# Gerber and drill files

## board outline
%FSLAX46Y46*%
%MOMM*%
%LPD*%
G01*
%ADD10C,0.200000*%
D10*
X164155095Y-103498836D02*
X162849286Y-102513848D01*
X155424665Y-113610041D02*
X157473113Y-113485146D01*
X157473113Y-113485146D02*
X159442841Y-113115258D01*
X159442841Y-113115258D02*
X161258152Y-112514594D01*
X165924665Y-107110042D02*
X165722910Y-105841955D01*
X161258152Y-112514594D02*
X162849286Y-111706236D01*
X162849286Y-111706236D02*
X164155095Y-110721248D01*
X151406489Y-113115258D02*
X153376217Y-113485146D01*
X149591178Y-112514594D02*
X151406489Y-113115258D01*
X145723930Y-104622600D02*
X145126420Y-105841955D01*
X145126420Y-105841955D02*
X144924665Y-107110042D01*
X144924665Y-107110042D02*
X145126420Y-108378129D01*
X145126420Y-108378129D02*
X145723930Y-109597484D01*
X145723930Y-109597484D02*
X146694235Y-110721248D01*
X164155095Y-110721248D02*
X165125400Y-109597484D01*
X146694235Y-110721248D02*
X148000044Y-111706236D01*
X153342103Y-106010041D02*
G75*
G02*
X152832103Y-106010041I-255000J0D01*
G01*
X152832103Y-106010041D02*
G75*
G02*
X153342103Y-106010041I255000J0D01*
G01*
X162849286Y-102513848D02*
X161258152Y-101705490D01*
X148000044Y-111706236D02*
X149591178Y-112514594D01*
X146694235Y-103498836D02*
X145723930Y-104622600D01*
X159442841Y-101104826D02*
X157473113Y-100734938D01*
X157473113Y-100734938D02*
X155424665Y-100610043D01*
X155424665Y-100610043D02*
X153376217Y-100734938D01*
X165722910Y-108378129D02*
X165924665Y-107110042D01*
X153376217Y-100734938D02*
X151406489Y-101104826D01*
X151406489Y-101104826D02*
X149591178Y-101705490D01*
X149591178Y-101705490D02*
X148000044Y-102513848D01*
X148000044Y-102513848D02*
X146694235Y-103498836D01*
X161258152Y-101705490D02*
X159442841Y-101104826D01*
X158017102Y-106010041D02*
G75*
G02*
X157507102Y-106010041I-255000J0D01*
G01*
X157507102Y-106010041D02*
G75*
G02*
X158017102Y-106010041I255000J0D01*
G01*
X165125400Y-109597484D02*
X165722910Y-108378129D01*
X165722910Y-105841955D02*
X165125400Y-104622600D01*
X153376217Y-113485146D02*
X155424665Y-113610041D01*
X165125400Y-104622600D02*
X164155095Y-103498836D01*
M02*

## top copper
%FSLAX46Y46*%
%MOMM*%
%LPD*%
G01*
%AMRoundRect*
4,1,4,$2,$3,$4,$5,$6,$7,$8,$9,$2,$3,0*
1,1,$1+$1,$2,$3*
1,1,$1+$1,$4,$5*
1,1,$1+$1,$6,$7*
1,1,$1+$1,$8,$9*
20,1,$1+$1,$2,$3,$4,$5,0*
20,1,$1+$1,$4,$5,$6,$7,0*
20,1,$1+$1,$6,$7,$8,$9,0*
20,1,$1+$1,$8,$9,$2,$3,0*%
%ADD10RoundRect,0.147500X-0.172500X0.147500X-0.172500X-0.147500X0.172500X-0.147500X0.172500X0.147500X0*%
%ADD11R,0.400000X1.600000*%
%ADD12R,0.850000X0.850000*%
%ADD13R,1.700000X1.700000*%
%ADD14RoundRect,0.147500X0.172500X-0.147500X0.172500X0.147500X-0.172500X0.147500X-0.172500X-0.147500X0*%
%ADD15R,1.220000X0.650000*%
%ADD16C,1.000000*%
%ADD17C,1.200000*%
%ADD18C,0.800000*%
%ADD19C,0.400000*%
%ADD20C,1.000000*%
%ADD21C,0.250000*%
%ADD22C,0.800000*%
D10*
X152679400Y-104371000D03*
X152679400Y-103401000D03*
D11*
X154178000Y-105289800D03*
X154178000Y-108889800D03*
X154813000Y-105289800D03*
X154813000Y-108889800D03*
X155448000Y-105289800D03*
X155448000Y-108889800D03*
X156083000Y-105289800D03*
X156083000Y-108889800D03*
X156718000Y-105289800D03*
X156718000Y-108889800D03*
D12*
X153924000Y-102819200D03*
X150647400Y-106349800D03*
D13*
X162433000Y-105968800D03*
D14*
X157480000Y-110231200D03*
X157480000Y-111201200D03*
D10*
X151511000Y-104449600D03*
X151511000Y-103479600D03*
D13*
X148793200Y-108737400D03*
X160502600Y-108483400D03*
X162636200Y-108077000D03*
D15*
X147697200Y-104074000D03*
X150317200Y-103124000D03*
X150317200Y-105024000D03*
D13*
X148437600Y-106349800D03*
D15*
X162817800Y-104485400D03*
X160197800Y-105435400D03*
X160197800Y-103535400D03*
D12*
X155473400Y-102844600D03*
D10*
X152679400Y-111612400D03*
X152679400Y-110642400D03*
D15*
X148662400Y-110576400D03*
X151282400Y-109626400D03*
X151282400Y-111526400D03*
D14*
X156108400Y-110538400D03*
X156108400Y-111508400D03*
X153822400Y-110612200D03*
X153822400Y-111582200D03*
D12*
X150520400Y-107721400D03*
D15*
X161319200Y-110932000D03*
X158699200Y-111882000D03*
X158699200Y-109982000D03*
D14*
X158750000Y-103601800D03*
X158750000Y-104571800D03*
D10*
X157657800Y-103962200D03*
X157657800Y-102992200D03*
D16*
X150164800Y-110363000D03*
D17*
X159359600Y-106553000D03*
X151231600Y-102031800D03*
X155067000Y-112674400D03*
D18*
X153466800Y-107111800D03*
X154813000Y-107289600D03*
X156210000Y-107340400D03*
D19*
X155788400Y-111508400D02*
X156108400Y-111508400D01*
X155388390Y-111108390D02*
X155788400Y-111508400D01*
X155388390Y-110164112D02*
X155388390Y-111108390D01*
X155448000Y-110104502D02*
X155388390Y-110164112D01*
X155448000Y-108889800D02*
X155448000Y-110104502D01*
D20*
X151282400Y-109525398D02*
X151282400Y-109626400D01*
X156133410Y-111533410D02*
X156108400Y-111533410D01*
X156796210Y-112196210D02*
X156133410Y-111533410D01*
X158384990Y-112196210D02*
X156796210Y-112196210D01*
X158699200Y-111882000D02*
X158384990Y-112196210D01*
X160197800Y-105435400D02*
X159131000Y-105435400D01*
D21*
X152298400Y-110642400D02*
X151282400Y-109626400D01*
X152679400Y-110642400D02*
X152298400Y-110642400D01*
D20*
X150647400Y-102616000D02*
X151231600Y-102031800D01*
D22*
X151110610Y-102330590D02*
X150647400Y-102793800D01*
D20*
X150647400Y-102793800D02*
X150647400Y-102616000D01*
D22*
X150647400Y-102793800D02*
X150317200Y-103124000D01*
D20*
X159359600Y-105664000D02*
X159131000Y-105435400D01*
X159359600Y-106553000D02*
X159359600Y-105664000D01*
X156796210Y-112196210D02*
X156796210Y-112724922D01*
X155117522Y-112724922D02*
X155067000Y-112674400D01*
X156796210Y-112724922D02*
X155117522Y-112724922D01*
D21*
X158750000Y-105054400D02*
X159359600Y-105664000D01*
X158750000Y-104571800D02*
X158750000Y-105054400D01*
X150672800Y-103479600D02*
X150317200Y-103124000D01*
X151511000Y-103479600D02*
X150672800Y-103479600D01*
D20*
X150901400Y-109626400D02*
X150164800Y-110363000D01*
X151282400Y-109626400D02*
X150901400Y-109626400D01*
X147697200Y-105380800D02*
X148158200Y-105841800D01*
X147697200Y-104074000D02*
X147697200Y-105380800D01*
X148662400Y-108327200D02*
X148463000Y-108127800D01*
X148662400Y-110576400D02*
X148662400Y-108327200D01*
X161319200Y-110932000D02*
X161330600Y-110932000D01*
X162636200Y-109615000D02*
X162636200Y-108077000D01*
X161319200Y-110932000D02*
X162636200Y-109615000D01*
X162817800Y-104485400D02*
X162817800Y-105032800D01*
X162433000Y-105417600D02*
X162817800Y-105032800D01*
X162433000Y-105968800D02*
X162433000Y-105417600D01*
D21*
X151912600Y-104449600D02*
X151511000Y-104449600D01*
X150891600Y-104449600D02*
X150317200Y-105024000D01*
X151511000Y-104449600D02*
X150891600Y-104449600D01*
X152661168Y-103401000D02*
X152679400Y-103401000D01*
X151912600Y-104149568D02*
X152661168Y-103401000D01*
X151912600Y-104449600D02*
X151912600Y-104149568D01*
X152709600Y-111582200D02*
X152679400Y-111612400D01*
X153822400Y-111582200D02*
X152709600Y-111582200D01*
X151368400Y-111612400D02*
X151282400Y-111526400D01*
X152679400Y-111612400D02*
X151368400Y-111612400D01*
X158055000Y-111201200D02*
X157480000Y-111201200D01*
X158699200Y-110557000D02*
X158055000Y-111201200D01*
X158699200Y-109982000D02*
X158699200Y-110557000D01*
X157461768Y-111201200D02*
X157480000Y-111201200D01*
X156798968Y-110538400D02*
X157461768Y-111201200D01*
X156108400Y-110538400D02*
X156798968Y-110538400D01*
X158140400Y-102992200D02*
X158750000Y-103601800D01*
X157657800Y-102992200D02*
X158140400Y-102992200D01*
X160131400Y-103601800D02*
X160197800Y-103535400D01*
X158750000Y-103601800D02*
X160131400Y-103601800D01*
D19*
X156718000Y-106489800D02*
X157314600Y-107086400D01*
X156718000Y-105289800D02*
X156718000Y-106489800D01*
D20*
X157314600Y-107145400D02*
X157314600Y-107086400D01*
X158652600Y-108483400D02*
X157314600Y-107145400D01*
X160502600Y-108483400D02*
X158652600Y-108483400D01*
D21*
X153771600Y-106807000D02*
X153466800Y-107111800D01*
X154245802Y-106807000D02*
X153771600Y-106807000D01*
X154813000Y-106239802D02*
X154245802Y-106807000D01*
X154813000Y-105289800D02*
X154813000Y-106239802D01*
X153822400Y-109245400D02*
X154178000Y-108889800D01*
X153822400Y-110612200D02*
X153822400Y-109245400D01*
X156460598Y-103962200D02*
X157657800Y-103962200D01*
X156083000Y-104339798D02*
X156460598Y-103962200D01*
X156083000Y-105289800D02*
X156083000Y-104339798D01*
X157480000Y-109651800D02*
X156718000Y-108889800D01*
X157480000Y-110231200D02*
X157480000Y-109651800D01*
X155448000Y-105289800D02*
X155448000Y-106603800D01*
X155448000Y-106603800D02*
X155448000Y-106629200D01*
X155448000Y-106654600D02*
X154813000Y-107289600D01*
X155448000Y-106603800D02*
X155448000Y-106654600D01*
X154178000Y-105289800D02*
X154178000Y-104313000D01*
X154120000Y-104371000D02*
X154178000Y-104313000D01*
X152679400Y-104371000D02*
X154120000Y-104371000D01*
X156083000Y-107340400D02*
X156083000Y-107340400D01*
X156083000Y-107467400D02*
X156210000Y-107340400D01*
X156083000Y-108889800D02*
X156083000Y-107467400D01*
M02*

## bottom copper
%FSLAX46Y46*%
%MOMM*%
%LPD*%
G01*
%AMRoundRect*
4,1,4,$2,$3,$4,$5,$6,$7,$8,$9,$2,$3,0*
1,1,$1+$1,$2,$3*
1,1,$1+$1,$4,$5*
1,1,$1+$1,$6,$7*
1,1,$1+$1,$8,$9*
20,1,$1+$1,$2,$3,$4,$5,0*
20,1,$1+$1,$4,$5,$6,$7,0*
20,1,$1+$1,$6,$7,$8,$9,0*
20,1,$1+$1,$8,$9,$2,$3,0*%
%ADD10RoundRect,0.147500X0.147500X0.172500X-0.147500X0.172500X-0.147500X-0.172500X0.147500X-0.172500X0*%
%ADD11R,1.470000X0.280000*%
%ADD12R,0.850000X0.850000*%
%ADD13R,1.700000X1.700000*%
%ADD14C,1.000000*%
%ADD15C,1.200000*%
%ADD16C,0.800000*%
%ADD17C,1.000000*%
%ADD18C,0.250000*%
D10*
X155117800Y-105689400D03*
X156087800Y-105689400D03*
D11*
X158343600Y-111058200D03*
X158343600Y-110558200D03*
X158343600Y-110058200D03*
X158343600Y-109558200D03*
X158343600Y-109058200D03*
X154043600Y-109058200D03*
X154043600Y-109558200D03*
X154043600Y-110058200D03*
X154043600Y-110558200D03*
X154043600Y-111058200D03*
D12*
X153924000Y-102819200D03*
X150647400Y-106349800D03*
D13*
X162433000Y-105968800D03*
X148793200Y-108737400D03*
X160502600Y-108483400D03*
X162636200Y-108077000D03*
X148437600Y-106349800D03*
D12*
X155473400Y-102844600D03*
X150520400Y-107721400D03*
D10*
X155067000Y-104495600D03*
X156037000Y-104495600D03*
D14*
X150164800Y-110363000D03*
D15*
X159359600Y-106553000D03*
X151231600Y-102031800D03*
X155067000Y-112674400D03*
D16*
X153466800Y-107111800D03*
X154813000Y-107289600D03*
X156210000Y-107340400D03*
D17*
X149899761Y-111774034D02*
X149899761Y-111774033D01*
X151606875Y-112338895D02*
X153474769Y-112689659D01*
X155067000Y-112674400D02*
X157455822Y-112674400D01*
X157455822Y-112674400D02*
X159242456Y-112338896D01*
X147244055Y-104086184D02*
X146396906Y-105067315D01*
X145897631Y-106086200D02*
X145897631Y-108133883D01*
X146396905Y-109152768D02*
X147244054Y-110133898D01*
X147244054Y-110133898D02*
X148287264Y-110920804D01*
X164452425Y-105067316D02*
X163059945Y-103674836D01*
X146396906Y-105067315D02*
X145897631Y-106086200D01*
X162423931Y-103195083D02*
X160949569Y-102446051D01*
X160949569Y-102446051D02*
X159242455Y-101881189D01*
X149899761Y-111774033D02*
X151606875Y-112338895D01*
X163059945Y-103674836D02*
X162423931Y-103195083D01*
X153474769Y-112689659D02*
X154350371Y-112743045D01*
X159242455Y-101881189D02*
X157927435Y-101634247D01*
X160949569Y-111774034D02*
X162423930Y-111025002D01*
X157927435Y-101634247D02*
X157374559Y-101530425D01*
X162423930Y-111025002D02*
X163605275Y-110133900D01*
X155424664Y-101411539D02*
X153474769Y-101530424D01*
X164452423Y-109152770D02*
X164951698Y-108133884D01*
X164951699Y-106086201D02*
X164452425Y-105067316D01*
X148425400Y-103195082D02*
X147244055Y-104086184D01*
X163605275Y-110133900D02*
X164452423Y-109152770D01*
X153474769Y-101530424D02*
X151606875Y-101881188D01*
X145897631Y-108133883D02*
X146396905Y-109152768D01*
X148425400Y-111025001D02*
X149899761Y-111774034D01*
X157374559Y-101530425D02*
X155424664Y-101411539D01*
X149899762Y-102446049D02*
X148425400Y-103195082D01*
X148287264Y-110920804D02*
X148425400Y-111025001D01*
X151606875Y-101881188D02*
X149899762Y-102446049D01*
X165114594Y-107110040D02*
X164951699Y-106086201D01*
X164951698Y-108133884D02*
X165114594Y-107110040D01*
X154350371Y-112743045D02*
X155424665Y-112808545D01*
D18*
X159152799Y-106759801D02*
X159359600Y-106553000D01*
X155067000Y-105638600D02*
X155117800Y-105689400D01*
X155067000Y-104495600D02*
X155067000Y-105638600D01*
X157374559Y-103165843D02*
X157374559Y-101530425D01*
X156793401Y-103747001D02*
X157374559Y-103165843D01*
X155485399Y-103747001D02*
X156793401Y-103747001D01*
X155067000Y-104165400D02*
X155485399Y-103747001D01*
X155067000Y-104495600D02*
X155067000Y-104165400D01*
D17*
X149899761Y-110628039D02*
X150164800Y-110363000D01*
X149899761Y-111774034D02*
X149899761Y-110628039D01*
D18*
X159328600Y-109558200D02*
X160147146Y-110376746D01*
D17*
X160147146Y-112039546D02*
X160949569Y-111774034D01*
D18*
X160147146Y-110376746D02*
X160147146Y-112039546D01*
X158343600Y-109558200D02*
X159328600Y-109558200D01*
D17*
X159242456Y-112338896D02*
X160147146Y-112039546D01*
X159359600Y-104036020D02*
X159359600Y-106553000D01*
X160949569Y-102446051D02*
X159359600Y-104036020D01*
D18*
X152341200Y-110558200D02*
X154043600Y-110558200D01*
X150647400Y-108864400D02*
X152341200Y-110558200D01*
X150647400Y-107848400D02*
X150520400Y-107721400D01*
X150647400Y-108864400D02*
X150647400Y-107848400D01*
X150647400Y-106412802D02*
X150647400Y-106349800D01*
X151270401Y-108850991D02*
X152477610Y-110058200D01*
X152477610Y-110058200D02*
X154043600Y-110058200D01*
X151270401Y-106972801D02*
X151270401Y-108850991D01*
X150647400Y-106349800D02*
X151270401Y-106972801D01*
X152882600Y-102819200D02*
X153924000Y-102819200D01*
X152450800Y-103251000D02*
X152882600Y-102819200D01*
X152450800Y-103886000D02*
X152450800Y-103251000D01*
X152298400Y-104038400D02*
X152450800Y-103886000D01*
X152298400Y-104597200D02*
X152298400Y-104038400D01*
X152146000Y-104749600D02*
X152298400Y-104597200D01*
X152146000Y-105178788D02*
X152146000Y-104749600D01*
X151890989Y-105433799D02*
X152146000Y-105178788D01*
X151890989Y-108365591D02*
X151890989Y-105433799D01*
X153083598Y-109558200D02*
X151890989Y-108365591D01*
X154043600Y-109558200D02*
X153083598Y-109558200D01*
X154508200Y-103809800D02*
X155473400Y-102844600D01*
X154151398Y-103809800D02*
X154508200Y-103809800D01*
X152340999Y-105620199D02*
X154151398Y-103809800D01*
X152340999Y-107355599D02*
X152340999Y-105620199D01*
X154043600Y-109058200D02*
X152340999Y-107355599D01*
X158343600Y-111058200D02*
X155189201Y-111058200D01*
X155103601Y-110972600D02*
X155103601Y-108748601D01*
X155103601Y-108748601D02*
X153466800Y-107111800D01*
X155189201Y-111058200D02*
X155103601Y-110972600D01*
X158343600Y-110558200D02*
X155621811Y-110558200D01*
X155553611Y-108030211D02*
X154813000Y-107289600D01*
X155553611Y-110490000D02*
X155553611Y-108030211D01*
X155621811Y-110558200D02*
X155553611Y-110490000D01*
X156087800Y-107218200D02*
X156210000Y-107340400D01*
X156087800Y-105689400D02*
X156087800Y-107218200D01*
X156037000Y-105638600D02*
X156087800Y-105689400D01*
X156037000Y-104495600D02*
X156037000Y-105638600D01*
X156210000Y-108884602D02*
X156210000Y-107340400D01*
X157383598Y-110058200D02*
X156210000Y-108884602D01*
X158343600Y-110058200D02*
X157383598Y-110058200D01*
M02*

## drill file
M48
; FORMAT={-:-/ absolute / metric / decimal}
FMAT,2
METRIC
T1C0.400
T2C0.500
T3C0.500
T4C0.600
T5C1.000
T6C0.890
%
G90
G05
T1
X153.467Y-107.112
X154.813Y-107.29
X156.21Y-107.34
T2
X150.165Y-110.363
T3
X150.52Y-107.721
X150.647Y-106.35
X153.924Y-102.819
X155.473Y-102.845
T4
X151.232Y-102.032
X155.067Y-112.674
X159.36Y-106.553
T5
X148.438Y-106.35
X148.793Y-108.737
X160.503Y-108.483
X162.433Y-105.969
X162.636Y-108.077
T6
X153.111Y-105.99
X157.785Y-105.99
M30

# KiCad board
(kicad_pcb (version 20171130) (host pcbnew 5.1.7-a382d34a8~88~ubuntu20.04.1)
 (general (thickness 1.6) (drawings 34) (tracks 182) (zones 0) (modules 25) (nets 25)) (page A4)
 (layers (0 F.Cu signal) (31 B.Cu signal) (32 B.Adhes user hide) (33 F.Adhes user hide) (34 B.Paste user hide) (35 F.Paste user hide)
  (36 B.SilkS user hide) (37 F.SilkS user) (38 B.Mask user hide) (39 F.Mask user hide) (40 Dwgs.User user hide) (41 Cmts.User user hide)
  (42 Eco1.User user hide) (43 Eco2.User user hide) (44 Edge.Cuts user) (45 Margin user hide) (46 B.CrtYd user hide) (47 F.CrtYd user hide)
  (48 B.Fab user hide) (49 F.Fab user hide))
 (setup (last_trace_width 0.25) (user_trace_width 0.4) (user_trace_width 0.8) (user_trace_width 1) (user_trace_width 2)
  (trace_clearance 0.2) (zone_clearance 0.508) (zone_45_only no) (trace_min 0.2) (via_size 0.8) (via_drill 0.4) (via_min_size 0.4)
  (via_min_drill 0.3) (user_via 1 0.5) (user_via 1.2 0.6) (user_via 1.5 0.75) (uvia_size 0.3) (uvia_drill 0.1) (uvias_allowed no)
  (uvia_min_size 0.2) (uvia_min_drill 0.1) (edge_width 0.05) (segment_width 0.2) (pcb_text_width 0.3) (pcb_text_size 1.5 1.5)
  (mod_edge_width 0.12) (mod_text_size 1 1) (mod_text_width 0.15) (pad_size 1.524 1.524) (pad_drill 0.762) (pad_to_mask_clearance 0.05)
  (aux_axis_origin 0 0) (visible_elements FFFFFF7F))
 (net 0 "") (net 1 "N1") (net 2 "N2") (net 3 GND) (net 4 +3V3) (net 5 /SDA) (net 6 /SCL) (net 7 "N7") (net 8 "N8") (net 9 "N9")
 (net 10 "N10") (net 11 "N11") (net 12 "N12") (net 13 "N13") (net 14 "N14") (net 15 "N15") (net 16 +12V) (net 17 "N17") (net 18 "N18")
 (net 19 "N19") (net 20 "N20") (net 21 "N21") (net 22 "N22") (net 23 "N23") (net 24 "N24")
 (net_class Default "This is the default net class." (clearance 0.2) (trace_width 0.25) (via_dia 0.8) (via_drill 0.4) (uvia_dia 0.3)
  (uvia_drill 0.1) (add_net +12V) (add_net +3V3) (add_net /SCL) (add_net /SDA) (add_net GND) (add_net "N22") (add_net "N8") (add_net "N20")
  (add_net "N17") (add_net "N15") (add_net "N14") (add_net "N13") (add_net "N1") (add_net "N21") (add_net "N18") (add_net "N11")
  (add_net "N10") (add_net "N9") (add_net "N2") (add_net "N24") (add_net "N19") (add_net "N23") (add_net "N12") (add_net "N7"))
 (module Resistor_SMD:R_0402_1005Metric (layer F.Cu) (at 152.6794 103.886 270)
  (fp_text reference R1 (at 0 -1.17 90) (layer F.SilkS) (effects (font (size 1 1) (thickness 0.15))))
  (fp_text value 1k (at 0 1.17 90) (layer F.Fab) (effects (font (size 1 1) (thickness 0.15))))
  (pad 2 smd roundrect (at 0.485 0 270) (size 0.59 0.64) (layers F.Cu F.Paste F.Mask) (roundrect_rratio 0.25) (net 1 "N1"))
  (pad 1 smd roundrect (at -0.485 0 270) (size 0.59 0.64) (layers F.Cu F.Paste F.Mask) (roundrect_rratio 0.25) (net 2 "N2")))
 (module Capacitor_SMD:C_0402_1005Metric (layer B.Cu) (at 155.6028 105.6894 180)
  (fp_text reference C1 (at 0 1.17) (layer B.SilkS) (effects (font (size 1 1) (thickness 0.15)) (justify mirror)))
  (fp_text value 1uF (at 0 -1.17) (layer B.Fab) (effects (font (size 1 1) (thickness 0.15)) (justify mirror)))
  (pad 2 smd roundrect (at 0.485 0 180) (size 0.59 0.64) (layers B.Cu B.Paste B.Mask) (roundrect_rratio 0.25) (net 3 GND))
  (pad 1 smd roundrect (at -0.485 0 180) (size 0.59 0.64) (layers B.Cu B.Paste B.Mask) (roundrect_rratio 0.25) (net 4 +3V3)))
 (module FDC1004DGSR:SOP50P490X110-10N (layer B.Cu) (at 156.1936 110.0582)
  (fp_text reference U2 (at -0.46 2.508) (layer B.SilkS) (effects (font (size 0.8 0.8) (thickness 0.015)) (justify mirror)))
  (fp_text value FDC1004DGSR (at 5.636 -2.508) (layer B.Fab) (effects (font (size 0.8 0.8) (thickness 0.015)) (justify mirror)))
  (pad 10 smd rect (at 2.15 1) (size 1.47 0.28) (layers B.Cu B.Paste B.Mask) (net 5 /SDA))
  (pad 9 smd rect (at 2.15 0.5) (size 1.47 0.28) (layers B.Cu B.Paste B.Mask) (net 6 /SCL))
  (pad 8 smd rect (at 2.15 0) (size 1.47 0.28) (layers B.Cu B.Paste B.Mask) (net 4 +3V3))
  (pad 7 smd rect (at 2.15 -0.5) (size 1.47 0.28) (layers B.Cu B.Paste B.Mask) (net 3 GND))
  (pad 6 smd rect (at 2.15 -1) (size 1.47 0.28) (layers B.Cu B.Paste B.Mask) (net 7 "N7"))
  (pad 5 smd rect (at -2.15 -1) (size 1.47 0.28) (layers B.Cu B.Paste B.Mask) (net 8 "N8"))
  (pad 4 smd rect (at -2.15 -0.5) (size 1.47 0.28) (layers B.Cu B.Paste B.Mask) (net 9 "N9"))
  (pad 3 smd rect (at -2.15 0) (size 1.47 0.28) (layers B.Cu B.Paste B.Mask) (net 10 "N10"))
  (pad 2 smd rect (at -2.15 0.5) (size 1.47 0.28) (layers B.Cu B.Paste B.Mask) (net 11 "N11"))
  (pad 1 smd rect (at -2.15 1) (size 1.47 0.28) (layers B.Cu B.Paste B.Mask) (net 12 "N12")))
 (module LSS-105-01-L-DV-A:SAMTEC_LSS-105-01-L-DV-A (layer F.Cu) (at 156.718 108.8898)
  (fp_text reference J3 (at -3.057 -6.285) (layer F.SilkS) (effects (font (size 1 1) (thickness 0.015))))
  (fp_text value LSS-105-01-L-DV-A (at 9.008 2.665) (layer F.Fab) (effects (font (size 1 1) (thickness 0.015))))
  (pad 10 smd rect (at -2.54 -3.6) (size 0.4 1.6) (layers F.Cu F.Paste F.Mask) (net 1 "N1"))
  (pad 09 smd rect (at -2.54 0) (size 0.4 1.6) (layers F.Cu F.Paste F.Mask) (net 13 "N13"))
  (pad 08 smd rect (at -1.905 -3.6) (size 0.4 1.6) (layers F.Cu F.Paste F.Mask) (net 5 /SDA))
  (pad 07 smd rect (at -1.905 0) (size 0.4 1.6) (layers F.Cu F.Paste F.Mask) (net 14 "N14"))
  (pad 06 smd rect (at -1.27 -3.6) (size 0.4 1.6) (layers F.Cu F.Paste F.Mask) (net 6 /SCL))
  (pad 05 smd rect (at -1.27 0) (size 0.4 1.6) (layers F.Cu F.Paste F.Mask) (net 3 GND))
  (pad 04 smd rect (at -0.635 -3.6) (size 0.4 1.6) (layers F.Cu F.Paste F.Mask) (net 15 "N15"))
  (pad 03 smd rect (at -0.635 0) (size 0.4 1.6) (layers F.Cu F.Paste F.Mask) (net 4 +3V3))
  (pad 02 smd rect (at 0 -3.6) (size 0.4 1.6) (layers F.Cu F.Paste F.Mask) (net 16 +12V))
  (pad 01 smd rect (at 0 0) (size 0.4 1.6) (layers F.Cu F.Paste F.Mask) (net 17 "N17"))
  (pad None np_thru_hole circle (at 1.067 -2.9) (size 0.89 0.89) (drill 0.89) (layers *.Cu *.Mask))
  (pad None np_thru_hole circle (at -3.607 -2.9) (size 0.89 0.89) (drill 0.89) (layers *.Cu *.Mask)))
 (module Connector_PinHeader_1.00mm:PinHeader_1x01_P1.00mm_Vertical (layer F.Cu) (at 153.924 102.8192)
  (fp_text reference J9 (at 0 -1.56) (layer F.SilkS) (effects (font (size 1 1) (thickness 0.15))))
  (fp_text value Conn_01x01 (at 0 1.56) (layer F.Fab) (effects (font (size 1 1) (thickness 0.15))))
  (pad 1 thru_hole rect (at 0 0) (size 0.85 0.85) (drill 0.5) (layers *.Cu *.Mask) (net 9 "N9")))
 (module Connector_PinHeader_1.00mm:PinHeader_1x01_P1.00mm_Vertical (layer F.Cu) (at 150.6474 106.3498)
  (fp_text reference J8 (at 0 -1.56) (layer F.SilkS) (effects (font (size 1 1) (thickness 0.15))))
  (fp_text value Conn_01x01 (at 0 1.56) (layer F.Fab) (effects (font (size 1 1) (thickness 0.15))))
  (pad 1 thru_hole rect (at 0 0) (size 0.85 0.85) (drill 0.5) (layers *.Cu *.Mask) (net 10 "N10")))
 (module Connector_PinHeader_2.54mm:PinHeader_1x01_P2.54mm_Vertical (layer F.Cu) (at 162.433 105.9688)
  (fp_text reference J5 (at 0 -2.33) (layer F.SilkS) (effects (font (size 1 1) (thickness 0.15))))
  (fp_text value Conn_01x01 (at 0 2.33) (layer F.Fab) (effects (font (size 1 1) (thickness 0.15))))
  (pad 1 thru_hole rect (at 0 0) (size 1.7 1.7) (drill 1) (layers *.Cu *.Mask) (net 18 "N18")))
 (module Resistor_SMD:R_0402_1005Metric (layer F.Cu) (at 157.48 110.7162 90)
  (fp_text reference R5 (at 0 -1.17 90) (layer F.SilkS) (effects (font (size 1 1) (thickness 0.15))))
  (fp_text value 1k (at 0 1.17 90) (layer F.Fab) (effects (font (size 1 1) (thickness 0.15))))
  (pad 2 smd roundrect (at 0.485 0 90) (size 0.59 0.64) (layers F.Cu F.Paste F.Mask) (roundrect_rratio 0.25) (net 17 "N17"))
  (pad 1 smd roundrect (at -0.485 0 90) (size 0.59 0.64) (layers F.Cu F.Paste F.Mask) (roundrect_rratio 0.25) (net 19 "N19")))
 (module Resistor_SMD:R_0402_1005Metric (layer F.Cu) (at 151.511 103.9646 270)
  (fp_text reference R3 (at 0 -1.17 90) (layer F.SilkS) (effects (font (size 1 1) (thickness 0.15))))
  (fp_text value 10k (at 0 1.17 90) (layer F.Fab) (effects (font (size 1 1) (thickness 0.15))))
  (pad 2 smd roundrect (at 0.485 0 270) (size 0.59 0.64) (layers F.Cu F.Paste F.Mask) (roundrect_rratio 0.25) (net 2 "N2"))
  (pad 1 smd roundrect (at -0.485 0 270) (size 0.59 0.64) (layers F.Cu F.Paste F.Mask) (roundrect_rratio 0.25) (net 3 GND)))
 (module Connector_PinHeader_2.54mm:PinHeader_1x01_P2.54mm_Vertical (layer F.Cu) (at 148.7932 108.7374)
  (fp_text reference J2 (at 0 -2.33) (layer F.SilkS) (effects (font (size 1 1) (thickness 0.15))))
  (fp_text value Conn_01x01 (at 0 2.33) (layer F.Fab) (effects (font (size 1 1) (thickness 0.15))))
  (pad 1 thru_hole rect (at 0 0) (size 1.7 1.7) (drill 1) (layers *.Cu *.Mask) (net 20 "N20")))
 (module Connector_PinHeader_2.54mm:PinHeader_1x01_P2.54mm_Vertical (layer F.Cu) (at 160.5026 108.4834)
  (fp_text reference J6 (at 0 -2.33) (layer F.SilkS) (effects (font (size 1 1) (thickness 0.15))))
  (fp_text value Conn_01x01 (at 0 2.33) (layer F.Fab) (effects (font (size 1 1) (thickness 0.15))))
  (pad 1 thru_hole rect (at 0 0) (size 1.7 1.7) (drill 1) (layers *.Cu *.Mask) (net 16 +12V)))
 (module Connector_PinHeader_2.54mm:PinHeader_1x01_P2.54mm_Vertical (layer F.Cu) (at 162.6362 108.077)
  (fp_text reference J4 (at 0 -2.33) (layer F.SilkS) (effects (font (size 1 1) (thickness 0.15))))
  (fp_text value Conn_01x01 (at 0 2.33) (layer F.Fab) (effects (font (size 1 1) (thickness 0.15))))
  (pad 1 thru_hole rect (at 0 0) (size 1.7 1.7) (drill 1) (layers *.Cu *.Mask) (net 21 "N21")))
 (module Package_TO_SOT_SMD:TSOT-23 (layer F.Cu) (at 149.0072 104.074 180)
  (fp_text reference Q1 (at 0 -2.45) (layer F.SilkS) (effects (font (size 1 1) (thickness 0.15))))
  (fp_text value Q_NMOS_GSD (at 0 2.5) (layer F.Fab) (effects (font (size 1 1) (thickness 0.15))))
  (pad 3 smd rect (at 1.31 0 180) (size 1.22 0.65) (layers F.Cu F.Paste F.Mask) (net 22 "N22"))
  (pad 2 smd rect (at -1.31 0.95 180) (size 1.22 0.65) (layers F.Cu F.Paste F.Mask) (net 3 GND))
  (pad 1 smd rect (at -1.31 -0.95 180) (size 1.22 0.65) (layers F.Cu F.Paste F.Mask) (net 2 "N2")))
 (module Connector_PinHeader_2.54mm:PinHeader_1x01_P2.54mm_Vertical (layer F.Cu) (at 148.4376 106.3498)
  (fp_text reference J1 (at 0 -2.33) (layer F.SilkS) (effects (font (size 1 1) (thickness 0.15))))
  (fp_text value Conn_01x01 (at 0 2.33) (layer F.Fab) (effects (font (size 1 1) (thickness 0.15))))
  (pad 1 thru_hole rect (at 0 0) (size 1.7 1.7) (drill 1) (layers *.Cu *.Mask) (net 22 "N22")))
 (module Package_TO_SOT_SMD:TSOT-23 (layer F.Cu) (at 161.5078 104.4854)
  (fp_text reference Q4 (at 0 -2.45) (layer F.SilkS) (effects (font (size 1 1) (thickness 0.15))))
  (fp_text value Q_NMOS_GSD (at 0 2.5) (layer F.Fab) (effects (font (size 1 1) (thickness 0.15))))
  (pad 3 smd rect (at 1.31 0) (size 1.22 0.65) (layers F.Cu F.Paste F.Mask) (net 18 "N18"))
  (pad 2 smd rect (at -1.31 0.95) (size 1.22 0.65) (layers F.Cu F.Paste F.Mask) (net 3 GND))
  (pad 1 smd rect (at -1.31 -0.95) (size 1.22 0.65) (layers F.Cu F.Paste F.Mask) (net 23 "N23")))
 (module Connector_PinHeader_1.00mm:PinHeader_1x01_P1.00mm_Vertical (layer F.Cu) (at 155.4734 102.8446)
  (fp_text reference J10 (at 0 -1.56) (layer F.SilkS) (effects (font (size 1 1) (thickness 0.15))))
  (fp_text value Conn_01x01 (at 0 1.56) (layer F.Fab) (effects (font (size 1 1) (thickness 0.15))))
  (pad 1 thru_hole rect (at 0 0) (size 0.85 0.85) (drill 0.5) (layers *.Cu *.Mask) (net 8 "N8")))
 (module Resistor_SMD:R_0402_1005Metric (layer F.Cu) (at 152.6794 111.1274 270)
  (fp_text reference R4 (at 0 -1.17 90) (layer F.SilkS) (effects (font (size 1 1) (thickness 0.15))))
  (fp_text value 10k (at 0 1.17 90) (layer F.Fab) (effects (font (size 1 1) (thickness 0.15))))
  (pad 2 smd roundrect (at 0.485 0 270) (size 0.59 0.64) (layers F.Cu F.Paste F.Mask) (roundrect_rratio 0.25) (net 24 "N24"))
  (pad 1 smd roundrect (at -0.485 0 270) (size 0.59 0.64) (layers F.Cu F.Paste F.Mask) (roundrect_rratio 0.25) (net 3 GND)))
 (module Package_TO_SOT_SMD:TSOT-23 (layer F.Cu) (at 149.9724 110.5764 180)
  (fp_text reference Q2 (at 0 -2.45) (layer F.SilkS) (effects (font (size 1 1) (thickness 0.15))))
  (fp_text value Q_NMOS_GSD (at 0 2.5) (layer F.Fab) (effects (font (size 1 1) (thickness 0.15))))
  (pad 3 smd rect (at 1.31 0 180) (size 1.22 0.65) (layers F.Cu F.Paste F.Mask) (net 20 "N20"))
  (pad 2 smd rect (at -1.31 0.95 180) (size 1.22 0.65) (layers F.Cu F.Paste F.Mask) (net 3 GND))
  (pad 1 smd rect (at -1.31 -0.95 180) (size 1.22 0.65) (layers F.Cu F.Paste F.Mask) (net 24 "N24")))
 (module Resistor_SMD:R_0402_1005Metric (layer F.Cu) (at 156.1084 111.0234 90)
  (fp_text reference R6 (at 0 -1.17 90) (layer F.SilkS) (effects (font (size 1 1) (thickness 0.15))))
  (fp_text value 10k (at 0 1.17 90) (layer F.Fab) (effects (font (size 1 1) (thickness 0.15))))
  (pad 2 smd roundrect (at 0.485 0 90) (size 0.59 0.64) (layers F.Cu F.Paste F.Mask) (roundrect_rratio 0.25) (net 19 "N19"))
  (pad 1 smd roundrect (at -0.485 0 90) (size 0.59 0.64) (layers F.Cu F.Paste F.Mask) (roundrect_rratio 0.25) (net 3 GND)))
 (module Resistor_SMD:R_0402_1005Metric (layer F.Cu) (at 153.8224 111.0972 90)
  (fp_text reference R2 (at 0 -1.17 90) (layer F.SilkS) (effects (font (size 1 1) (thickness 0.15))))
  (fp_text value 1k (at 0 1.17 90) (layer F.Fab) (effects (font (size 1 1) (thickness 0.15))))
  (pad 2 smd roundrect (at 0.485 0 90) (size 0.59 0.64) (layers F.Cu F.Paste F.Mask) (roundrect_rratio 0.25) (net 13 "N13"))
  (pad 1 smd roundrect (at -0.485 0 90) (size 0.59 0.64) (layers F.Cu F.Paste F.Mask) (roundrect_rratio 0.25) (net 24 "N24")))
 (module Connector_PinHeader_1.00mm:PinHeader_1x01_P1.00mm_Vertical (layer F.Cu) (at 150.5204 107.7214)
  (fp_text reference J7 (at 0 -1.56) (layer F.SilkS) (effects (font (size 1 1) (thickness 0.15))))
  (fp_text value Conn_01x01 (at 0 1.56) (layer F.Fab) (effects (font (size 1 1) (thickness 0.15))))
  (pad 1 thru_hole rect (at 0 0) (size 0.85 0.85) (drill 0.5) (layers *.Cu *.Mask) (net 11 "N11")))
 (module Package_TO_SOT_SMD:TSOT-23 (layer F.Cu) (at 160.0092 110.932)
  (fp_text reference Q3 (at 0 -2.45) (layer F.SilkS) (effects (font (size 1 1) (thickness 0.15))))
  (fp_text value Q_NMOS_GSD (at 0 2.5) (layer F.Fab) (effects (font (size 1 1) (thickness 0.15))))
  (pad 3 smd rect (at 1.31 0) (size 1.22 0.65) (layers F.Cu F.Paste F.Mask) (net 21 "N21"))
  (pad 2 smd rect (at -1.31 0.95) (size 1.22 0.65) (layers F.Cu F.Paste F.Mask) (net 3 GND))
  (pad 1 smd rect (at -1.31 -0.95) (size 1.22 0.65) (layers F.Cu F.Paste F.Mask) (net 19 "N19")))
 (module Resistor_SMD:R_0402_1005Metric (layer F.Cu) (at 158.75 104.0868 90)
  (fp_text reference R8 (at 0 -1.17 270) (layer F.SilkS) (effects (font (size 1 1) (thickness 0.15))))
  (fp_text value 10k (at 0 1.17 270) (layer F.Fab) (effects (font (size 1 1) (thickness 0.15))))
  (pad 2 smd roundrect (at 0.485 0 90) (size 0.59 0.64) (layers F.Cu F.Paste F.Mask) (roundrect_rratio 0.25) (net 23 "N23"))
  (pad 1 smd roundrect (at -0.485 0 90) (size 0.59 0.64) (layers F.Cu F.Paste F.Mask) (roundrect_rratio 0.25) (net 3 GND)))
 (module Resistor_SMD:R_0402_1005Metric (layer F.Cu) (at 157.6578 103.4772 270)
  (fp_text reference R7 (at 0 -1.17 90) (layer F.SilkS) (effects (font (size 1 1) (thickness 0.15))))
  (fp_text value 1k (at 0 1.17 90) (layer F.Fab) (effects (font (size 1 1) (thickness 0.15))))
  (pad 2 smd roundrect (at 0.485 0 270) (size 0.59 0.64) (layers F.Cu F.Paste F.Mask) (roundrect_rratio 0.25) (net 15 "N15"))
  (pad 1 smd roundrect (at -0.485 0 270) (size 0.59 0.64) (layers F.Cu F.Paste F.Mask) (roundrect_rratio 0.25) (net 23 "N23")))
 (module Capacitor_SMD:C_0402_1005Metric (layer B.Cu) (at 155.552 104.4956 180)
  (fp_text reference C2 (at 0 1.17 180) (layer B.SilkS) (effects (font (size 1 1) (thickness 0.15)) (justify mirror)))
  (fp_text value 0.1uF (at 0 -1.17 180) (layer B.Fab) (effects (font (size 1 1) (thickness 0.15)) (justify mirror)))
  (pad 2 smd roundrect (at 0.485 0 180) (size 0.59 0.64) (layers B.Cu B.Paste B.Mask) (roundrect_rratio 0.25) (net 3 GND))
  (pad 1 smd roundrect (at -0.485 0 180) (size 0.59 0.64) (layers B.Cu B.Paste B.Mask) (roundrect_rratio 0.25) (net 4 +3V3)))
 (gr_line (start 164.155095 103.498836) (end 162.849286 102.513848) (layer Edge.Cuts) (width 0.2))
 (gr_line (start 155.424665 113.610041) (end 157.473113 113.485146) (layer Edge.Cuts) (width 0.2))
 (gr_line (start 157.473113 113.485146) (end 159.442841 113.115258) (layer Edge.Cuts) (width 0.2))
 (gr_line (start 159.442841 113.115258) (end 161.258152 112.514594) (layer Edge.Cuts) (width 0.2))
 (gr_line (start 165.924665 107.110042) (end 165.72291 105.841955) (layer Edge.Cuts) (width 0.2))
 (gr_line (start 161.258152 112.514594) (end 162.849286 111.706236) (layer Edge.Cuts) (width 0.2))
 (gr_line (start 162.849286 111.706236) (end 164.155095 110.721248) (layer Edge.Cuts) (width 0.2))
 (gr_line (start 151.406489 113.115258) (end 153.376217 113.485146) (layer Edge.Cuts) (width 0.2))
 (gr_line (start 149.591178 112.514594) (end 151.406489 113.115258) (layer Edge.Cuts) (width 0.2))
 (gr_line (start 145.72393 104.6226) (end 145.12642 105.841955) (layer Edge.Cuts) (width 0.2))
 (gr_line (start 145.12642 105.841955) (end 144.924665 107.110042) (layer Edge.Cuts) (width 0.2))
 (gr_line (start 144.924665 107.110042) (end 145.12642 108.378129) (layer Edge.Cuts) (width 0.2))
 (gr_line (start 145.12642 108.378129) (end 145.72393 109.597484) (layer Edge.Cuts) (width 0.2))
 (gr_line (start 145.72393 109.597484) (end 146.694235 110.721248) (layer Edge.Cuts) (width 0.2))
 (gr_line (start 164.155095 110.721248) (end 165.1254 109.597484) (layer Edge.Cuts) (width 0.2))
 (gr_line (start 146.694235 110.721248) (end 148.000044 111.706236) (layer Edge.Cuts) (width 0.2))
 (gr_circle (center 153.087103 106.010041) (end 153.342103 106.010041) (layer Edge.Cuts) (width 0.2))
 (gr_line (start 162.849286 102.513848) (end 161.258152 101.70549) (layer Edge.Cuts) (width 0.2))
 (gr_line (start 148.000044 111.706236) (end 149.591178 112.514594) (layer Edge.Cuts) (width 0.2))
 (gr_line (start 146.694235 103.498836) (end 145.72393 104.6226) (layer Edge.Cuts) (width 0.2))
 (gr_line (start 159.442841 101.104826) (end 157.473113 100.734938) (layer Edge.Cuts) (width 0.2))
 (gr_line (start 157.473113 100.734938) (end 155.424665 100.610043) (layer Edge.Cuts) (width 0.2))
 (gr_line (start 155.424665 100.610043) (end 153.376217 100.734938) (layer Edge.Cuts) (width 0.2))
 (gr_line (start 165.72291 108.378129) (end 165.924665 107.110042) (layer Edge.Cuts) (width 0.2))
 (gr_line (start 153.376217 100.734938) (end 151.406489 101.104826) (layer Edge.Cuts) (width 0.2))
 (gr_line (start 151.406489 101.104826) (end 149.591178 101.70549) (layer Edge.Cuts) (width 0.2))
 (gr_line (start 149.591178 101.70549) (end 148.000044 102.513848) (layer Edge.Cuts) (width 0.2))
 (gr_line (start 148.000044 102.513848) (end 146.694235 103.498836) (layer Edge.Cuts) (width 0.2))
 (gr_line (start 161.258152 101.70549) (end 159.442841 101.104826) (layer Edge.Cuts) (width 0.2))
 (gr_circle (center 157.762102 106.010041) (end 158.017102 106.010041) (layer Edge.Cuts) (width 0.2))
 (gr_line (start 165.1254 109.597484) (end 165.72291 108.378129) (layer Edge.Cuts) (width 0.2))
 (gr_line (start 165.72291 105.841955) (end 165.1254 104.6226) (layer Edge.Cuts) (width 0.2))
 (gr_line (start 153.376217 113.485146) (end 155.424665 113.610041) (layer Edge.Cuts) (width 0.2))
 (gr_line (start 165.1254 104.6226) (end 164.155095 103.498836) (layer Edge.Cuts) (width 0.2))
 (via (at 150.1648 110.363) (size 1) (drill 0.5) (layers F.Cu B.Cu) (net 3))
 (via (at 159.3596 106.553) (size 1.2) (drill 0.6) (layers F.Cu B.Cu) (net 3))
 (via (at 151.2316 102.0318) (size 1.2) (drill 0.6) (layers F.Cu B.Cu) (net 3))
 (via (at 155.067 112.6744) (size 1.2) (drill 0.6) (layers F.Cu B.Cu) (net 3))
 (segment (start 155.7884 111.5084) (end 156.1084 111.5084) (width 0.4) (layer F.Cu) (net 3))
 (segment (start 155.38839 111.10839) (end 155.7884 111.5084) (width 0.4) (layer F.Cu) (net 3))
 (segment (start 155.38839 110.164112) (end 155.38839 111.10839) (width 0.4) (layer F.Cu) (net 3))
 (segment (start 155.448 110.104502) (end 155.38839 110.164112) (width 0.4) (layer F.Cu) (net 3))
 (segment (start 155.448 108.8898) (end 155.448 110.104502) (width 0.4) (layer F.Cu) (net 3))
 (segment (start 151.2824 109.525398) (end 151.2824 109.6264) (width 1) (layer F.Cu) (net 3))
 (segment (start 156.13341 111.53341) (end 156.1084 111.53341) (width 1) (layer F.Cu) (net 3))
 (segment (start 156.79621 112.19621) (end 156.13341 111.53341) (width 1) (layer F.Cu) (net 3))
 (segment (start 158.38499 112.19621) (end 156.79621 112.19621) (width 1) (layer F.Cu) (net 3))
 (segment (start 158.6992 111.882) (end 158.38499 112.19621) (width 1) (layer F.Cu) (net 3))
 (segment (start 160.1978 105.4354) (end 159.131 105.4354) (width 1) (layer F.Cu) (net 3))
 (segment (start 152.2984 110.6424) (end 151.2824 109.6264) (width 0.25) (layer F.Cu) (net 3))
 (segment (start 152.6794 110.6424) (end 152.2984 110.6424) (width 0.25) (layer F.Cu) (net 3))
 (segment (start 149.899761 111.774034) (end 149.899761 111.774033) (width 1) (layer B.Cu) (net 3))
 (segment (start 151.606875 112.338895) (end 153.474769 112.689659) (width 1) (layer B.Cu) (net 3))
 (segment (start 155.067 112.6744) (end 157.455822 112.6744) (width 1) (layer B.Cu) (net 3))
 (segment (start 157.455822 112.6744) (end 159.242456 112.338896) (width 1) (layer B.Cu) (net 3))
 (segment (start 147.244055 104.086184) (end 146.396906 105.067315) (width 1) (layer B.Cu) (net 3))
 (segment (start 145.897631 106.0862) (end 145.897631 108.133883) (width 1) (layer B.Cu) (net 3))
 (segment (start 146.396905 109.152768) (end 147.244054 110.133898) (width 1) (layer B.Cu) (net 3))
 (segment (start 147.244054 110.133898) (end 148.287264 110.920804) (width 1) (layer B.Cu) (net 3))
 (segment (start 164.452425 105.067316) (end 163.059945 103.674836) (width 1) (layer B.Cu) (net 3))
 (segment (start 146.396906 105.067315) (end 145.897631 106.0862) (width 1) (layer B.Cu) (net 3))
 (segment (start 162.423931 103.195083) (end 160.949569 102.446051) (width 1) (layer B.Cu) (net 3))
 (segment (start 160.949569 102.446051) (end 159.242455 101.881189) (width 1) (layer B.Cu) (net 3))
 (segment (start 149.899761 111.774033) (end 151.606875 112.338895) (width 1) (layer B.Cu) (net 3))
 (segment (start 163.059945 103.674836) (end 162.423931 103.195083) (width 1) (layer B.Cu) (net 3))
 (segment (start 153.474769 112.689659) (end 154.350371 112.743045) (width 1) (layer B.Cu) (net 3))
 (segment (start 159.242455 101.881189) (end 157.927435 101.634247) (width 1) (layer B.Cu) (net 3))
 (segment (start 160.949569 111.774034) (end 162.42393 111.025002) (width 1) (layer B.Cu) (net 3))
 (segment (start 157.927435 101.634247) (end 157.374559 101.530425) (width 1) (layer B.Cu) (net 3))
 (segment (start 162.42393 111.025002) (end 163.605275 110.1339) (width 1) (layer B.Cu) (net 3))
 (segment (start 155.424664 101.411539) (end 153.474769 101.530424) (width 1) (layer B.Cu) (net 3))
 (segment (start 164.452423 109.15277) (end 164.951698 108.133884) (width 1) (layer B.Cu) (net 3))
 (segment (start 164.951699 106.086201) (end 164.452425 105.067316) (width 1) (layer B.Cu) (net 3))
 (segment (start 148.4254 103.195082) (end 147.244055 104.086184) (width 1) (layer B.Cu) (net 3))
 (segment (start 163.605275 110.1339) (end 164.452423 109.15277) (width 1) (layer B.Cu) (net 3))
 (segment (start 153.474769 101.530424) (end 151.606875 101.881188) (width 1) (layer B.Cu) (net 3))
 (segment (start 145.897631 108.133883) (end 146.396905 109.152768) (width 1) (layer B.Cu) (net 3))
 (segment (start 148.4254 111.025001) (end 149.899761 111.774034) (width 1) (layer B.Cu) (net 3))
 (segment (start 157.374559 101.530425) (end 155.424664 101.411539) (width 1) (layer B.Cu) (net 3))
 (segment (start 149.899762 102.446049) (end 148.4254 103.195082) (width 1) (layer B.Cu) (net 3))
 (segment (start 148.287264 110.920804) (end 148.4254 111.025001) (width 1) (layer B.Cu) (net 3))
 (segment (start 151.606875 101.881188) (end 149.899762 102.446049) (width 1) (layer B.Cu) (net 3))
 (segment (start 165.114594 107.11004) (end 164.951699 106.086201) (width 1) (layer B.Cu) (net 3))
 (segment (start 164.951698 108.133884) (end 165.114594 107.11004) (width 1) (layer B.Cu) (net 3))
 (segment (start 154.350371 112.743045) (end 155.424665 112.808545) (width 1) (layer B.Cu) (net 3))
 (segment (start 150.6474 102.616) (end 151.2316 102.0318) (width 1) (layer F.Cu) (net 3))
 (segment (start 151.11061 102.33059) (end 150.6474 102.7938) (width 0.8) (layer F.Cu) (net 3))
 (segment (start 150.6474 102.7938) (end 150.6474 102.616) (width 1) (layer F.Cu) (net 3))
 (segment (start 150.6474 102.7938) (end 150.3172 103.124) (width 0.8) (layer F.Cu) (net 3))
 (segment (start 159.3596 105.664) (end 159.131 105.4354) (width 1) (layer F.Cu) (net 3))
 (segment (start 159.3596 106.553) (end 159.3596 105.664) (width 1) (layer F.Cu) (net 3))
 (segment (start 156.79621 112.19621) (end 156.79621 112.724922) (width 1) (layer F.Cu) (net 3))
 (segment (start 155.117522 112.724922) (end 155.067 112.6744) (width 1) (layer F.Cu) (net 3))
 (segment (start 156.79621 112.724922) (end 155.117522 112.724922) (width 1) (layer F.Cu) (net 3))
 (segment (start 158.75 105.0544) (end 159.3596 105.664) (width 0.25) (layer F.Cu) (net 3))
 (segment (start 158.75 104.5718) (end 158.75 105.0544) (width 0.25) (layer F.Cu) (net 3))
 (segment (start 150.6728 103.4796) (end 150.3172 103.124) (width 0.25) (layer F.Cu) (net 3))
 (segment (start 151.511 103.4796) (end 150.6728 103.4796) (width 0.25) (layer F.Cu) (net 3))
 (segment (start 159.152799 106.759801) (end 159.3596 106.553) (width 0.25) (layer B.Cu) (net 3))
 (segment (start 155.067 105.6386) (end 155.1178 105.6894) (width 0.25) (layer B.Cu) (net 3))
 (segment (start 155.067 104.4956) (end 155.067 105.6386) (width 0.25) (layer B.Cu) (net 3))
 (segment (start 157.374559 103.165843) (end 157.374559 101.530425) (width 0.25) (layer B.Cu) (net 3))
 (segment (start 156.793401 103.747001) (end 157.374559 103.165843) (width 0.25) (layer B.Cu) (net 3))
 (segment (start 155.485399 103.747001) (end 156.793401 103.747001) (width 0.25) (layer B.Cu) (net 3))
 (segment (start 155.067 104.1654) (end 155.485399 103.747001) (width 0.25) (layer B.Cu) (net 3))
 (segment (start 155.067 104.4956) (end 155.067 104.1654) (width 0.25) (layer B.Cu) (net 3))
 (segment (start 150.9014 109.6264) (end 150.1648 110.363) (width 1) (layer F.Cu) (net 3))
 (segment (start 151.2824 109.6264) (end 150.9014 109.6264) (width 1) (layer F.Cu) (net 3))
 (segment (start 149.899761 110.628039) (end 150.1648 110.363) (width 1) (layer B.Cu) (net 3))
 (segment (start 149.899761 111.774034) (end 149.899761 110.628039) (width 1) (layer B.Cu) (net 3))
 (segment (start 159.3286 109.5582) (end 160.147146 110.376746) (width 0.25) (layer B.Cu) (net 3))
 (segment (start 160.147146 112.039546) (end 160.949569 111.774034) (width 1) (layer B.Cu) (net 3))
 (segment (start 160.147146 110.376746) (end 160.147146 112.039546) (width 0.25) (layer B.Cu) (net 3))
 (segment (start 158.3436 109.5582) (end 159.3286 109.5582) (width 0.25) (layer B.Cu) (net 3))
 (segment (start 159.242456 112.338896) (end 160.147146 112.039546) (width 1) (layer B.Cu) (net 3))
 (segment (start 159.3596 104.03602) (end 159.3596 106.553) (width 1) (layer B.Cu) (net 3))
 (segment (start 160.949569 102.446051) (end 159.3596 104.03602) (width 1) (layer B.Cu) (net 3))
 (segment (start 147.6972 105.3808) (end 148.1582 105.8418) (width 1) (layer F.Cu) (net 22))
 (segment (start 147.6972 104.074) (end 147.6972 105.3808) (width 1) (layer F.Cu) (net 22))
 (segment (start 148.6624 108.3272) (end 148.463 108.1278) (width 1) (layer F.Cu) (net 20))
 (segment (start 148.6624 110.5764) (end 148.6624 108.3272) (width 1) (layer F.Cu) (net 20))
 (segment (start 161.3192 110.932) (end 161.3306 110.932) (width 1) (layer F.Cu) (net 21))
 (segment (start 162.6362 109.615) (end 162.6362 108.077) (width 1) (layer F.Cu) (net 21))
 (segment (start 161.3192 110.932) (end 162.6362 109.615) (width 1) (layer F.Cu) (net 21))
 (segment (start 162.8178 104.4854) (end 162.8178 105.0328) (width 1) (layer F.Cu) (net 18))
 (segment (start 162.433 105.4176) (end 162.8178 105.0328) (width 1) (layer F.Cu) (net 18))
 (segment (start 162.433 105.9688) (end 162.433 105.4176) (width 1) (layer F.Cu) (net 18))
 (segment (start 151.9126 104.4496) (end 151.511 104.4496) (width 0.25) (layer F.Cu) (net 2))
 (segment (start 150.8916 104.4496) (end 150.3172 105.024) (width 0.25) (layer F.Cu) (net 2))
 (segment (start 151.511 104.4496) (end 150.8916 104.4496) (width 0.25) (layer F.Cu) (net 2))
 (segment (start 152.661168 103.401) (end 152.6794 103.401) (width 0.25) (layer F.Cu) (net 2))
 (segment (start 151.9126 104.149568) (end 152.661168 103.401) (width 0.25) (layer F.Cu) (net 2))
 (segment (start 151.9126 104.4496) (end 151.9126 104.149568) (width 0.25) (layer F.Cu) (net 2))
 (segment (start 152.7096 111.5822) (end 152.6794 111.6124) (width 0.25) (layer F.Cu) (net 24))
 (segment (start 153.8224 111.5822) (end 152.7096 111.5822) (width 0.25) (layer F.Cu) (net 24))
 (segment (start 151.3684 111.6124) (end 151.2824 111.5264) (width 0.25) (layer F.Cu) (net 24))
 (segment (start 152.6794 111.6124) (end 151.3684 111.6124) (width 0.25) (layer F.Cu) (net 24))
 (segment (start 158.055 111.2012) (end 157.48 111.2012) (width 0.25) (layer F.Cu) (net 19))
 (segment (start 158.6992 110.557) (end 158.055 111.2012) (width 0.25) (layer F.Cu) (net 19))
 (segment (start 158.6992 109.982) (end 158.6992 110.557) (width 0.25) (layer F.Cu) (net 19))
 (segment (start 157.461768 111.2012) (end 157.48 111.2012) (width 0.25) (layer F.Cu) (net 19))
 (segment (start 156.798968 110.5384) (end 157.461768 111.2012) (width 0.25) (layer F.Cu) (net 19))
 (segment (start 156.1084 110.5384) (end 156.798968 110.5384) (width 0.25) (layer F.Cu) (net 19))
 (segment (start 158.1404 102.9922) (end 158.75 103.6018) (width 0.25) (layer F.Cu) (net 23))
 (segment (start 157.6578 102.9922) (end 158.1404 102.9922) (width 0.25) (layer F.Cu) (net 23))
 (segment (start 160.1314 103.6018) (end 160.1978 103.5354) (width 0.25) (layer F.Cu) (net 23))
 (segment (start 158.75 103.6018) (end 160.1314 103.6018) (width 0.25) (layer F.Cu) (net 23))
 (segment (start 156.718 106.4898) (end 157.3146 107.0864) (width 0.4) (layer F.Cu) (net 16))
 (segment (start 156.718 105.2898) (end 156.718 106.4898) (width 0.4) (layer F.Cu) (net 16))
 (segment (start 157.3146 107.1454) (end 157.3146 107.0864) (width 1) (layer F.Cu) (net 16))
 (segment (start 158.6526 108.4834) (end 157.3146 107.1454) (width 1) (layer F.Cu) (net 16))
 (segment (start 160.5026 108.4834) (end 158.6526 108.4834) (width 1) (layer F.Cu) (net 16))
 (segment (start 152.3412 110.5582) (end 154.0436 110.5582) (width 0.25) (layer B.Cu) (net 11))
 (segment (start 150.6474 108.8644) (end 152.3412 110.5582) (width 0.25) (layer B.Cu) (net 11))
 (segment (start 150.6474 107.8484) (end 150.5204 107.7214) (width 0.25) (layer B.Cu) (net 11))
 (segment (start 150.6474 108.8644) (end 150.6474 107.8484) (width 0.25) (layer B.Cu) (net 11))
 (segment (start 150.6474 106.412802) (end 150.6474 106.3498) (width 0.25) (layer B.Cu) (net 10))
 (segment (start 151.270401 108.850991) (end 152.47761 110.0582) (width 0.25) (layer B.Cu) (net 10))
 (segment (start 152.47761 110.0582) (end 154.0436 110.0582) (width 0.25) (layer B.Cu) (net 10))
 (segment (start 151.270401 106.972801) (end 151.270401 108.850991) (width 0.25) (layer B.Cu) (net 10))
 (segment (start 150.6474 106.3498) (end 151.270401 106.972801) (width 0.25) (layer B.Cu) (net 10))
 (segment (start 152.8826 102.8192) (end 153.924 102.8192) (width 0.25) (layer B.Cu) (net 9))
 (segment (start 152.4508 103.251) (end 152.8826 102.8192) (width 0.25) (layer B.Cu) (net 9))
 (segment (start 152.4508 103.886) (end 152.4508 103.251) (width 0.25) (layer B.Cu) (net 9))
 (segment (start 152.2984 104.0384) (end 152.4508 103.886) (width 0.25) (layer B.Cu) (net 9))
 (segment (start 152.2984 104.5972) (end 152.2984 104.0384) (width 0.25) (layer B.Cu) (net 9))
 (segment (start 152.146 104.7496) (end 152.2984 104.5972) (width 0.25) (layer B.Cu) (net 9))
 (segment (start 152.146 105.178788) (end 152.146 104.7496) (width 0.25) (layer B.Cu) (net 9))
 (segment (start 151.890989 105.433799) (end 152.146 105.178788) (width 0.25) (layer B.Cu) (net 9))
 (segment (start 151.890989 108.365591) (end 151.890989 105.433799) (width 0.25) (layer B.Cu) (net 9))
 (segment (start 153.083598 109.5582) (end 151.890989 108.365591) (width 0.25) (layer B.Cu) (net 9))
 (segment (start 154.0436 109.5582) (end 153.083598 109.5582) (width 0.25) (layer B.Cu) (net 9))
 (segment (start 154.5082 103.8098) (end 155.4734 102.8446) (width 0.25) (layer B.Cu) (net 8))
 (segment (start 154.151398 103.8098) (end 154.5082 103.8098) (width 0.25) (layer B.Cu) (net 8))
 (segment (start 152.340999 105.620199) (end 154.151398 103.8098) (width 0.25) (layer B.Cu) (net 8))
 (segment (start 152.340999 107.355599) (end 152.340999 105.620199) (width 0.25) (layer B.Cu) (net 8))
 (segment (start 154.0436 109.0582) (end 152.340999 107.355599) (width 0.25) (layer B.Cu) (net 8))
 (via (at 153.4668 107.1118) (size 0.8) (drill 0.4) (layers F.Cu B.Cu) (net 5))
 (segment (start 153.7716 106.807) (end 153.4668 107.1118) (width 0.25) (layer F.Cu) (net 5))
 (segment (start 154.245802 106.807) (end 153.7716 106.807) (width 0.25) (layer F.Cu) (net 5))
 (segment (start 154.813 106.239802) (end 154.245802 106.807) (width 0.25) (layer F.Cu) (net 5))
 (segment (start 154.813 105.2898) (end 154.813 106.239802) (width 0.25) (layer F.Cu) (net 5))
 (segment (start 158.3436 111.0582) (end 155.189201 111.0582) (width 0.25) (layer B.Cu) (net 5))
 (segment (start 155.103601 110.9726) (end 155.103601 108.748601) (width 0.25) (layer B.Cu) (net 5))
 (segment (start 155.103601 108.748601) (end 153.4668 107.1118) (width 0.25) (layer B.Cu) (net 5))
 (segment (start 155.189201 111.0582) (end 155.103601 110.9726) (width 0.25) (layer B.Cu) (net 5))
 (segment (start 153.8224 109.2454) (end 154.178 108.8898) (width 0.25) (layer F.Cu) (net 13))
 (segment (start 153.8224 110.6122) (end 153.8224 109.2454) (width 0.25) (layer F.Cu) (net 13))
 (segment (start 156.460598 103.9622) (end 157.6578 103.9622) (width 0.25) (layer F.Cu) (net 15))
 (segment (start 156.083 104.339798) (end 156.460598 103.9622) (width 0.25) (layer F.Cu) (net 15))
 (segment (start 156.083 105.2898) (end 156.083 104.339798) (width 0.25) (layer F.Cu) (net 15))
 (segment (start 157.48 109.6518) (end 156.718 108.8898) (width 0.25) (layer F.Cu) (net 17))
 (segment (start 157.48 110.2312) (end 157.48 109.6518) (width 0.25) (layer F.Cu) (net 17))
 (via (at 154.813 107.2896) (size 0.8) (drill 0.4) (layers F.Cu B.Cu) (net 6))
 (segment (start 155.448 105.2898) (end 155.448 106.6038) (width 0.25) (layer F.Cu) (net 6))
 (segment (start 155.448 106.6038) (end 155.448 106.6292) (width 0.25) (layer F.Cu) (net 6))
 (segment (start 155.448 106.6546) (end 154.813 107.2896) (width 0.25) (layer F.Cu) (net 6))
 (segment (start 155.448 106.6038) (end 155.448 106.6546) (width 0.25) (layer F.Cu) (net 6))
 (segment (start 158.3436 110.5582) (end 155.621811 110.5582) (width 0.25) (layer B.Cu) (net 6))
 (segment (start 155.553611 108.030211) (end 154.813 107.2896) (width 0.25) (layer B.Cu) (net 6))
 (segment (start 155.553611 110.49) (end 155.553611 108.030211) (width 0.25) (layer B.Cu) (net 6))
 (segment (start 155.621811 110.5582) (end 155.553611 110.49) (width 0.25) (layer B.Cu) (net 6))
 (segment (start 154.178 105.2898) (end 154.178 104.313) (width 0.25) (layer F.Cu) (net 1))
 (segment (start 154.12 104.371) (end 154.178 104.313) (width 0.25) (layer F.Cu) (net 1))
 (segment (start 152.6794 104.371) (end 154.12 104.371) (width 0.25) (layer F.Cu) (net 1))
 (segment (start 156.083 107.3404) (end 156.083 107.3404) (width 0.25) (layer F.Cu) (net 4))
 (via (at 156.21 107.3404) (size 0.8) (drill 0.4) (layers F.Cu B.Cu) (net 4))
 (segment (start 156.083 107.4674) (end 156.21 107.3404) (width 0.25) (layer F.Cu) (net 4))
 (segment (start 156.083 108.8898) (end 156.083 107.4674) (width 0.25) (layer F.Cu) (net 4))
 (segment (start 156.0878 107.2182) (end 156.21 107.3404) (width 0.25) (layer B.Cu) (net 4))
 (segment (start 156.0878 105.6894) (end 156.0878 107.2182) (width 0.25) (layer B.Cu) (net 4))
 (segment (start 156.037 105.6386) (end 156.0878 105.6894) (width 0.25) (layer B.Cu) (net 4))
 (segment (start 156.037 104.4956) (end 156.037 105.6386) (width 0.25) (layer B.Cu) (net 4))
 (segment (start 156.21 108.884602) (end 156.21 107.3404) (width 0.25) (layer B.Cu) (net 4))
 (segment (start 157.383598 110.0582) (end 156.21 108.884602) (width 0.25) (layer B.Cu) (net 4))
 (segment (start 158.3436 110.0582) (end 157.383598 110.0582) (width 0.25) (layer B.Cu) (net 4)))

